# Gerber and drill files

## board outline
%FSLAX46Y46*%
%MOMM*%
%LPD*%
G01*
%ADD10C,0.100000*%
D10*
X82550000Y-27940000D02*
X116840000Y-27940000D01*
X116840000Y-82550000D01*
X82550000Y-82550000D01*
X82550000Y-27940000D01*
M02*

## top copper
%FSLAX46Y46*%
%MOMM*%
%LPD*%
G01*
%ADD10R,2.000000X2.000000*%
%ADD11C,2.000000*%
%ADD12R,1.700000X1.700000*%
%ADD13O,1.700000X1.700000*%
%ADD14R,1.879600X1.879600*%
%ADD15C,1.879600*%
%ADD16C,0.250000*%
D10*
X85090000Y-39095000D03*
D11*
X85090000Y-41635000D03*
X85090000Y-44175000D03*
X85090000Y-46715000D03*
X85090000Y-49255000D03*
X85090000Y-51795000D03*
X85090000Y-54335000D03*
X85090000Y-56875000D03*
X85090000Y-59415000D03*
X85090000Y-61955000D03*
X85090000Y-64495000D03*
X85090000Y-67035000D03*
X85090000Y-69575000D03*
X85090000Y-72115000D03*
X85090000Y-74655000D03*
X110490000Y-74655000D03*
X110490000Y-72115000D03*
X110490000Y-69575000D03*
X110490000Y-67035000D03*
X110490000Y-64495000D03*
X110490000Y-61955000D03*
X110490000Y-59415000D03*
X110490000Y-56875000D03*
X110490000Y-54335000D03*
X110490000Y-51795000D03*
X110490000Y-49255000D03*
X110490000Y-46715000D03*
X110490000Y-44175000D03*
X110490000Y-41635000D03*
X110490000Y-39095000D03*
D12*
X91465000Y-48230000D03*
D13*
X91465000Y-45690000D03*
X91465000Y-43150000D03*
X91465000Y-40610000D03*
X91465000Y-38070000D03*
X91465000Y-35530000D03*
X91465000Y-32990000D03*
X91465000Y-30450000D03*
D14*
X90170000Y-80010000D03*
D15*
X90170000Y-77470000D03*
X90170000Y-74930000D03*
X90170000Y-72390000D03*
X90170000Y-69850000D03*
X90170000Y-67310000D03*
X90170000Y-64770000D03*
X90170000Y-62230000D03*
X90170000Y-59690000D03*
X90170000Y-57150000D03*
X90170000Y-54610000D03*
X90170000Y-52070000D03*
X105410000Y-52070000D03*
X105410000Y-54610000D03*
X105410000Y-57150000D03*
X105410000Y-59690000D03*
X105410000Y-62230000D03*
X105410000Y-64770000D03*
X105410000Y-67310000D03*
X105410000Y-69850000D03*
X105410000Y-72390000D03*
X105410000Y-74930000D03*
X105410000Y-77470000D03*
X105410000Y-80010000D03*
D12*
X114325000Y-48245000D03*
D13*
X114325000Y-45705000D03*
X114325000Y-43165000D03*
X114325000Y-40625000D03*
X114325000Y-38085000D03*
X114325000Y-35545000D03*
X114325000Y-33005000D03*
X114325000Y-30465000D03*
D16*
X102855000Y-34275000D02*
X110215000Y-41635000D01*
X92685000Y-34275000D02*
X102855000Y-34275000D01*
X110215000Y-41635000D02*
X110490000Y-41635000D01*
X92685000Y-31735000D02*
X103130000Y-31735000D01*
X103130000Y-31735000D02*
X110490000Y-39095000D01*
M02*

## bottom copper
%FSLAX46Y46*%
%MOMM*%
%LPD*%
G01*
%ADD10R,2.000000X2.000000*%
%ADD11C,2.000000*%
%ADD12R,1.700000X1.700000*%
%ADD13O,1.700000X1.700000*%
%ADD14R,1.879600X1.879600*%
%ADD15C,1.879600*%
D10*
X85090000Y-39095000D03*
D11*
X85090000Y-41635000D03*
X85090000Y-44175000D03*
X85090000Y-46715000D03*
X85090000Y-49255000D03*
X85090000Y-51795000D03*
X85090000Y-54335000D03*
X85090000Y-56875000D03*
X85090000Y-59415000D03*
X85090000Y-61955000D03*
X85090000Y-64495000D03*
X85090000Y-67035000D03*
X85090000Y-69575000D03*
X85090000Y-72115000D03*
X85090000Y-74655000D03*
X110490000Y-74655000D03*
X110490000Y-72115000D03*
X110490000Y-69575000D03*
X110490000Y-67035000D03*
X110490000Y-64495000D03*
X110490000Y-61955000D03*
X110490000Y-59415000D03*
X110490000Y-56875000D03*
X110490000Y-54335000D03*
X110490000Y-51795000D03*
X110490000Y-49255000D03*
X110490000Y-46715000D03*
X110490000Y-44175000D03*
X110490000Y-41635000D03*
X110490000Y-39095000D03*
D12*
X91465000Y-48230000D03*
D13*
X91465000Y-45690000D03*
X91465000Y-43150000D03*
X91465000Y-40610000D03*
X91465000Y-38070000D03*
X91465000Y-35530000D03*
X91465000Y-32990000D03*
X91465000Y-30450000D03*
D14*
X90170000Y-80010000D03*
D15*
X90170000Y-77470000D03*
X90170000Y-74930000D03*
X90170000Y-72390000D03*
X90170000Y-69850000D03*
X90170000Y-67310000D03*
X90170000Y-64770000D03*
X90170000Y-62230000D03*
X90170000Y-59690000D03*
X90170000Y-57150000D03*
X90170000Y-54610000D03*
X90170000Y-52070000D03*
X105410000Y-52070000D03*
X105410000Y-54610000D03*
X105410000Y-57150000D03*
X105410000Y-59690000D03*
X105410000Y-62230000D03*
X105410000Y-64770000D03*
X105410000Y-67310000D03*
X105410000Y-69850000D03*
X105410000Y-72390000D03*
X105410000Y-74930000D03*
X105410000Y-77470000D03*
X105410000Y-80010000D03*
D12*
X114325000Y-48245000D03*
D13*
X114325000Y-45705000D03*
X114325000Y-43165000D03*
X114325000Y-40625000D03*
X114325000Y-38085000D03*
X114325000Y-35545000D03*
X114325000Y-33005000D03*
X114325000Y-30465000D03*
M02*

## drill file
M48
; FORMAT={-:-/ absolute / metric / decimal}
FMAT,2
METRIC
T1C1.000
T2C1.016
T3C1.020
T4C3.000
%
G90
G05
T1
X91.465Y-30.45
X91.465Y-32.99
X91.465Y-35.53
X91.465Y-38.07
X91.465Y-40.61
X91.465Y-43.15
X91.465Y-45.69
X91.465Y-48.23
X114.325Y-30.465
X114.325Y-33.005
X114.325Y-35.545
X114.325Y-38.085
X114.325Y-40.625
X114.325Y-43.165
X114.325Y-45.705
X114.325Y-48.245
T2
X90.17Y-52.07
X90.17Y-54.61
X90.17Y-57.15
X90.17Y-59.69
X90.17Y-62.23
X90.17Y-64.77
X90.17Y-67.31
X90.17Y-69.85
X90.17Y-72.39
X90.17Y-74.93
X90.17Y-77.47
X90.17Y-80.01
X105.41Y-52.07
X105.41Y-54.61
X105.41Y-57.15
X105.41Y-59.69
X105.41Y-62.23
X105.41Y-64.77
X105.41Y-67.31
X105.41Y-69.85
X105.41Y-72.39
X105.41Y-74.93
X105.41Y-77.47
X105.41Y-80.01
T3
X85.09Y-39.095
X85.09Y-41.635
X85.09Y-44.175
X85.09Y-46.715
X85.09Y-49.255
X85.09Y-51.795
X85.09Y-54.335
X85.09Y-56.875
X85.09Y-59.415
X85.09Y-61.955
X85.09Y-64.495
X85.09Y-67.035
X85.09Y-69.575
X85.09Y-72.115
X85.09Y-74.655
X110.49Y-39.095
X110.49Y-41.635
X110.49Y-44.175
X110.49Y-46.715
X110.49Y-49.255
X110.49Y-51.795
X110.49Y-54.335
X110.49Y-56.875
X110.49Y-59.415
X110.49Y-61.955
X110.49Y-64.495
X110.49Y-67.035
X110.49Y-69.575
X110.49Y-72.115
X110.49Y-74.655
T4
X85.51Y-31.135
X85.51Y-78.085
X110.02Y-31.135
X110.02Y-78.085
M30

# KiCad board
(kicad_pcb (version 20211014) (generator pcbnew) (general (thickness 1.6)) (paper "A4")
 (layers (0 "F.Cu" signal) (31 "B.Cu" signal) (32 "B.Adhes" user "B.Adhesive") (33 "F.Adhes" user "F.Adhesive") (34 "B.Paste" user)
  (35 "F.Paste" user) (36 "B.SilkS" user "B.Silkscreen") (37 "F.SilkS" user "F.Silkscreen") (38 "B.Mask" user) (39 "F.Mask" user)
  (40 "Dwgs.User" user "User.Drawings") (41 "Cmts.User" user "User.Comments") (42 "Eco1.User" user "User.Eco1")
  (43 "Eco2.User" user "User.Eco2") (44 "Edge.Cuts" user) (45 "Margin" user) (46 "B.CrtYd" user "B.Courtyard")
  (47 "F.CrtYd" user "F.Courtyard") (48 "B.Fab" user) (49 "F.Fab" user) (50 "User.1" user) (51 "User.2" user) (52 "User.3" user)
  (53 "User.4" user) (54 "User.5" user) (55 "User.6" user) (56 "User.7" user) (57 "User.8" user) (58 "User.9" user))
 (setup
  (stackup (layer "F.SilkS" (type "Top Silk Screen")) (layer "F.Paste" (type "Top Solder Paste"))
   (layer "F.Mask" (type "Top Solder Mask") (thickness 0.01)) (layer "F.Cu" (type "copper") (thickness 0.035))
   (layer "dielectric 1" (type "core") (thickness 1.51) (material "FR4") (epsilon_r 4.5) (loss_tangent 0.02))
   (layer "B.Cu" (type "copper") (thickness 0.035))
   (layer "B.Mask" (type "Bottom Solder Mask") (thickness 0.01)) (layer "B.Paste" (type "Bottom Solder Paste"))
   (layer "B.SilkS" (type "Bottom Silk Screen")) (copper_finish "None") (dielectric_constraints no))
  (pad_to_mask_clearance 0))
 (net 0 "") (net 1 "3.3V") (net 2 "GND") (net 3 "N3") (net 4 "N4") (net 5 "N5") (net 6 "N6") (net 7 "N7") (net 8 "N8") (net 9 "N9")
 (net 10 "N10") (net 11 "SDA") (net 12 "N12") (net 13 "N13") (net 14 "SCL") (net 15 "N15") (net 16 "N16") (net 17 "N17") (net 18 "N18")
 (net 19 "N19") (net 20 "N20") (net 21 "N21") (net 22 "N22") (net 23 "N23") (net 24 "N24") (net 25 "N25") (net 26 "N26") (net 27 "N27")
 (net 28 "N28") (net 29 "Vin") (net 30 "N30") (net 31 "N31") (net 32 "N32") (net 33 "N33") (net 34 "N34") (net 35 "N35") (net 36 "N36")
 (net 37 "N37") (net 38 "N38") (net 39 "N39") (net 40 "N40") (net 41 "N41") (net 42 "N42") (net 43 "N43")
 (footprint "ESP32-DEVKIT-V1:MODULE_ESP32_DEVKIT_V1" (layer "F.Cu") (at 97.79 54.61)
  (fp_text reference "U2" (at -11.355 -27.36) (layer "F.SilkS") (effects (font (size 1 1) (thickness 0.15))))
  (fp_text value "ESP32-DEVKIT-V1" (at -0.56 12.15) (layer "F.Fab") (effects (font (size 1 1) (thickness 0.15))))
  (pad "" np_thru_hole circle (at -12.28 23.475) (size 3 3) (drill 3) (layers *.Cu *.Mask))
  (pad "" np_thru_hole circle (at -12.28 -23.475) (size 3 3) (drill 3) (layers *.Cu *.Mask))
  (pad "" np_thru_hole circle (at 12.23 -23.475) (size 3 3) (drill 3) (layers *.Cu *.Mask))
  (pad "" np_thru_hole circle (at 12.23 23.475) (size 3 3) (drill 3) (layers *.Cu *.Mask))
  (pad "1" thru_hole rect (at -12.7 -15.515) (size 2 2) (drill 1.02) (layers *.Cu *.Mask) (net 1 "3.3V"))
  (pad "2" thru_hole circle (at -12.7 -12.975) (size 2 2) (drill 1.02) (layers *.Cu *.Mask) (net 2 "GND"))
  (pad "3" thru_hole circle (at -12.7 -10.435) (size 2 2) (drill 1.02) (layers *.Cu *.Mask) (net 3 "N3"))
  (pad "4" thru_hole circle (at -12.7 -7.895) (size 2 2) (drill 1.02) (layers *.Cu *.Mask) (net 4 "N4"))
  (pad "5" thru_hole circle (at -12.7 -5.355) (size 2 2) (drill 1.02) (layers *.Cu *.Mask) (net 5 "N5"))
  (pad "6" thru_hole circle (at -12.7 -2.815) (size 2 2) (drill 1.02) (layers *.Cu *.Mask) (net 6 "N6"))
  (pad "7" thru_hole circle (at -12.7 -0.275) (size 2 2) (drill 1.02) (layers *.Cu *.Mask) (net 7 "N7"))
  (pad "8" thru_hole circle (at -12.7 2.265) (size 2 2) (drill 1.02) (layers *.Cu *.Mask) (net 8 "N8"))
  (pad "9" thru_hole circle (at -12.7 4.805) (size 2 2) (drill 1.02) (layers *.Cu *.Mask) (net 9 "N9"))
  (pad "10" thru_hole circle (at -12.7 7.345) (size 2 2) (drill 1.02) (layers *.Cu *.Mask) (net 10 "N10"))
  (pad "11" thru_hole circle (at -12.7 9.885) (size 2 2) (drill 1.02) (layers *.Cu *.Mask) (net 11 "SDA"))
  (pad "12" thru_hole circle (at -12.7 12.425) (size 2 2) (drill 1.02) (layers *.Cu *.Mask) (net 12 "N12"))
  (pad "13" thru_hole circle (at -12.7 14.965) (size 2 2) (drill 1.02) (layers *.Cu *.Mask) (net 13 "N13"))
  (pad "14" thru_hole circle (at -12.7 17.505) (size 2 2) (drill 1.02) (layers *.Cu *.Mask) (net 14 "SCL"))
  (pad "15" thru_hole circle (at -12.7 20.045) (size 2 2) (drill 1.02) (layers *.Cu *.Mask) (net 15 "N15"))
  (pad "16" thru_hole circle (at 12.7 20.045) (size 2 2) (drill 1.02) (layers *.Cu *.Mask) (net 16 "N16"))
  (pad "17" thru_hole circle (at 12.7 17.505) (size 2 2) (drill 1.02) (layers *.Cu *.Mask) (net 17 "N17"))
  (pad "18" thru_hole circle (at 12.7 14.965) (size 2 2) (drill 1.02) (layers *.Cu *.Mask) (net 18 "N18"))
  (pad "19" thru_hole circle (at 12.7 12.425) (size 2 2) (drill 1.02) (layers *.Cu *.Mask) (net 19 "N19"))
  (pad "20" thru_hole circle (at 12.7 9.885) (size 2 2) (drill 1.02) (layers *.Cu *.Mask) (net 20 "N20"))
  (pad "21" thru_hole circle (at 12.7 7.345) (size 2 2) (drill 1.02) (layers *.Cu *.Mask) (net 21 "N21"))
  (pad "22" thru_hole circle (at 12.7 4.805) (size 2 2) (drill 1.02) (layers *.Cu *.Mask) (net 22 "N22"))
  (pad "23" thru_hole circle (at 12.7 2.265) (size 2 2) (drill 1.02) (layers *.Cu *.Mask) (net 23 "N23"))
  (pad "24" thru_hole circle (at 12.7 -0.275) (size 2 2) (drill 1.02) (layers *.Cu *.Mask) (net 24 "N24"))
  (pad "25" thru_hole circle (at 12.7 -2.815) (size 2 2) (drill 1.02) (layers *.Cu *.Mask) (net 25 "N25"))
  (pad "26" thru_hole circle (at 12.7 -5.355) (size 2 2) (drill 1.02) (layers *.Cu *.Mask) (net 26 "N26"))
  (pad "27" thru_hole circle (at 12.7 -7.895) (size 2 2) (drill 1.02) (layers *.Cu *.Mask) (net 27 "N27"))
  (pad "28" thru_hole circle (at 12.7 -10.435) (size 2 2) (drill 1.02) (layers *.Cu *.Mask) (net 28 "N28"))
  (pad "29" thru_hole circle (at 12.7 -12.975) (size 2 2) (drill 1.02) (layers *.Cu *.Mask) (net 2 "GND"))
  (pad "30" thru_hole circle (at 12.7 -15.515) (size 2 2) (drill 1.02) (layers *.Cu *.Mask) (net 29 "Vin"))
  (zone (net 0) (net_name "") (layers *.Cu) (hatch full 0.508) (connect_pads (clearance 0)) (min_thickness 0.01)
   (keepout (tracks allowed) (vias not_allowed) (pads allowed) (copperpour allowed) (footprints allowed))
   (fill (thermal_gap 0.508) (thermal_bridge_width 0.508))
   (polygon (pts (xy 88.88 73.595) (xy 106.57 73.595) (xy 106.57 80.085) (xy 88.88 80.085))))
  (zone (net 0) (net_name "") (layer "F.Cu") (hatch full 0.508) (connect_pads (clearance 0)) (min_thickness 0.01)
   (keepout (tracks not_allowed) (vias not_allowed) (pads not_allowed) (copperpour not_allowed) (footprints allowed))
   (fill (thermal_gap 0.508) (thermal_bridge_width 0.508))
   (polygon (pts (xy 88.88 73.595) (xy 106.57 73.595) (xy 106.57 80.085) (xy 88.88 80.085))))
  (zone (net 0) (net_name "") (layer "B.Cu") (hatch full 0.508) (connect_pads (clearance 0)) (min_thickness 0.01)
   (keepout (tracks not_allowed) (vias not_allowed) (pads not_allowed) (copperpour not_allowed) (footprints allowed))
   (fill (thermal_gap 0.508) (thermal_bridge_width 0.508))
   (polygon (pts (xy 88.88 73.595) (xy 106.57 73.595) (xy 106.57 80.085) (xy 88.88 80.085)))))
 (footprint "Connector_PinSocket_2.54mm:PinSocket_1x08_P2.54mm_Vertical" (layer "B.Cu") (at 91.465 48.23)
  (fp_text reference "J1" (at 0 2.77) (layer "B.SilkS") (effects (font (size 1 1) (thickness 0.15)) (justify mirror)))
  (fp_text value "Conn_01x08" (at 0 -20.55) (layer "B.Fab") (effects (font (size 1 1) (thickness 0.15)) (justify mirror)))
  (pad "1" thru_hole rect (at 0 0) (size 1.7 1.7) (drill 1) (layers *.Cu *.Mask) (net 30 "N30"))
  (pad "2" thru_hole oval (at 0 -2.54) (size 1.7 1.7) (drill 1) (layers *.Cu *.Mask) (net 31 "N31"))
  (pad "3" thru_hole oval (at 0 -5.08) (size 1.7 1.7) (drill 1) (layers *.Cu *.Mask) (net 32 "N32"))
  (pad "4" thru_hole oval (at 0 -7.62) (size 1.7 1.7) (drill 1) (layers *.Cu *.Mask) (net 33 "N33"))
  (pad "5" thru_hole oval (at 0 -10.16) (size 1.7 1.7) (drill 1) (layers *.Cu *.Mask) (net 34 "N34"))
  (pad "6" thru_hole oval (at 0 -12.7) (size 1.7 1.7) (drill 1) (layers *.Cu *.Mask) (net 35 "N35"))
  (pad "7" thru_hole oval (at 0 -15.24) (size 1.7 1.7) (drill 1) (layers *.Cu *.Mask) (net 2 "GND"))
  (pad "8" thru_hole oval (at 0 -17.78) (size 1.7 1.7) (drill 1) (layers *.Cu *.Mask) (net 29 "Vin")))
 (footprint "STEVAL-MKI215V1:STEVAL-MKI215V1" (layer "B.Cu") (at 97.79 66.04)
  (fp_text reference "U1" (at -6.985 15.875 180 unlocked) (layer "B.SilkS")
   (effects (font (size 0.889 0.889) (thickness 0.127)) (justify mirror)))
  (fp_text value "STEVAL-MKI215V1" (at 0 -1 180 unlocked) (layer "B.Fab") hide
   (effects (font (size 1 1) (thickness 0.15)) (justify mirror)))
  (pad "1" thru_hole rect (at -7.62 13.97) (size 1.8796 1.8796) (drill 1.016) (layers *.Cu *.Mask) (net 1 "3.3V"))
  (pad "2" thru_hole circle (at -7.62 11.43) (size 1.8796 1.8796) (drill 1.016) (layers *.Cu *.Mask))
  (pad "3" thru_hole circle (at -7.62 8.89) (size 1.8796 1.8796) (drill 1.016) (layers *.Cu *.Mask))
  (pad "4" thru_hole circle (at -7.62 6.35) (size 1.8796 1.8796) (drill 1.016) (layers *.Cu *.Mask))
  (pad "5" thru_hole circle (at -7.62 3.81) (size 1.8796 1.8796) (drill 1.016) (layers *.Cu *.Mask))
  (pad "6" thru_hole circle (at -7.62 1.27) (size 1.8796 1.8796) (drill 1.016) (layers *.Cu *.Mask))
  (pad "7" thru_hole circle (at -7.62 -1.27) (size 1.8796 1.8796) (drill 1.016) (layers *.Cu *.Mask))
  (pad "8" thru_hole circle (at -7.62 -3.81) (size 1.8796 1.8796) (drill 1.016) (layers *.Cu *.Mask))
  (pad "9" thru_hole circle (at -7.62 -6.35) (size 1.8796 1.8796) (drill 1.016) (layers *.Cu *.Mask))
  (pad "10" thru_hole circle (at -7.62 -8.89) (size 1.8796 1.8796) (drill 1.016) (layers *.Cu *.Mask))
  (pad "11" thru_hole circle (at -7.62 -11.43) (size 1.8796 1.8796) (drill 1.016) (layers *.Cu *.Mask))
  (pad "12" thru_hole circle (at -7.62 -13.97) (size 1.8796 1.8796) (drill 1.016) (layers *.Cu *.Mask))
  (pad "13" thru_hole circle (at 7.62 -13.97) (size 1.8796 1.8796) (drill 1.016) (layers *.Cu *.Mask) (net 2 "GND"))
  (pad "14" thru_hole circle (at 7.62 -11.43) (size 1.8796 1.8796) (drill 1.016) (layers *.Cu *.Mask))
  (pad "15" thru_hole circle (at 7.62 -8.89) (size 1.8796 1.8796) (drill 1.016) (layers *.Cu *.Mask))
  (pad "16" thru_hole circle (at 7.62 -6.35) (size 1.8796 1.8796) (drill 1.016) (layers *.Cu *.Mask))
  (pad "17" thru_hole circle (at 7.62 -3.81) (size 1.8796 1.8796) (drill 1.016) (layers *.Cu *.Mask))
  (pad "18" thru_hole circle (at 7.62 -1.27) (size 1.8796 1.8796) (drill 1.016) (layers *.Cu *.Mask))
  (pad "19" thru_hole circle (at 7.62 1.27) (size 1.8796 1.8796) (drill 1.016) (layers *.Cu *.Mask))
  (pad "20" thru_hole circle (at 7.62 3.81) (size 1.8796 1.8796) (drill 1.016) (layers *.Cu *.Mask) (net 14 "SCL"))
  (pad "21" thru_hole circle (at 7.62 6.35) (size 1.8796 1.8796) (drill 1.016) (layers *.Cu *.Mask) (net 11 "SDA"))
  (pad "22" thru_hole circle (at 7.62 8.89) (size 1.8796 1.8796) (drill 1.016) (layers *.Cu *.Mask) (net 1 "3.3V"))
  (pad "23" thru_hole circle (at 7.62 11.43) (size 1.8796 1.8796) (drill 1.016) (layers *.Cu *.Mask))
  (pad "24" thru_hole circle (at 7.62 13.97) (size 1.8796 1.8796) (drill 1.016) (layers *.Cu *.Mask)))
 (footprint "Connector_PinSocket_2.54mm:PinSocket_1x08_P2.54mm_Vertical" (layer "B.Cu") (at 114.325 48.245)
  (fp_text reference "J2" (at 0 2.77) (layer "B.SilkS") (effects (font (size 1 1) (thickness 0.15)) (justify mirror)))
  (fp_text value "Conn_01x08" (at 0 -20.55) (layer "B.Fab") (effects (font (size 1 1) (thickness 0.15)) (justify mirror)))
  (pad "1" thru_hole rect (at 0 0) (size 1.7 1.7) (drill 1) (layers *.Cu *.Mask) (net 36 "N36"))
  (pad "2" thru_hole oval (at 0 -2.54) (size 1.7 1.7) (drill 1) (layers *.Cu *.Mask) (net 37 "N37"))
  (pad "3" thru_hole oval (at 0 -5.08) (size 1.7 1.7) (drill 1) (layers *.Cu *.Mask) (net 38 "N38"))
  (pad "4" thru_hole oval (at 0 -7.62) (size 1.7 1.7) (drill 1) (layers *.Cu *.Mask) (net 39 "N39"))
  (pad "5" thru_hole oval (at 0 -10.16) (size 1.7 1.7) (drill 1) (layers *.Cu *.Mask) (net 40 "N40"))
  (pad "6" thru_hole oval (at 0 -12.7) (size 1.7 1.7) (drill 1) (layers *.Cu *.Mask) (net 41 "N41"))
  (pad "7" thru_hole oval (at 0 -15.24) (size 1.7 1.7) (drill 1) (layers *.Cu *.Mask) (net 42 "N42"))
  (pad "8" thru_hole oval (at 0 -17.78) (size 1.7 1.7) (drill 1) (layers *.Cu *.Mask) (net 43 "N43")))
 (gr_rect (start 82.55 27.94) (end 116.84 82.55) (layer "Edge.Cuts") (width 0.1) (fill none))
 (segment (start 102.855 34.275) (end 110.215 41.635) (width 0.25) (layer "F.Cu") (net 2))
 (segment (start 92.685 34.275) (end 102.855 34.275) (width 0.25) (layer "F.Cu") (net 2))
 (segment (start 110.215 41.635) (end 110.49 41.635) (width 0.25) (layer "F.Cu") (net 2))
 (segment (start 92.685 31.735) (end 103.13 31.735) (width 0.25) (layer "F.Cu") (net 29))
 (segment (start 103.13 31.735) (end 110.49 39.095) (width 0.25) (layer "F.Cu") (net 29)))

